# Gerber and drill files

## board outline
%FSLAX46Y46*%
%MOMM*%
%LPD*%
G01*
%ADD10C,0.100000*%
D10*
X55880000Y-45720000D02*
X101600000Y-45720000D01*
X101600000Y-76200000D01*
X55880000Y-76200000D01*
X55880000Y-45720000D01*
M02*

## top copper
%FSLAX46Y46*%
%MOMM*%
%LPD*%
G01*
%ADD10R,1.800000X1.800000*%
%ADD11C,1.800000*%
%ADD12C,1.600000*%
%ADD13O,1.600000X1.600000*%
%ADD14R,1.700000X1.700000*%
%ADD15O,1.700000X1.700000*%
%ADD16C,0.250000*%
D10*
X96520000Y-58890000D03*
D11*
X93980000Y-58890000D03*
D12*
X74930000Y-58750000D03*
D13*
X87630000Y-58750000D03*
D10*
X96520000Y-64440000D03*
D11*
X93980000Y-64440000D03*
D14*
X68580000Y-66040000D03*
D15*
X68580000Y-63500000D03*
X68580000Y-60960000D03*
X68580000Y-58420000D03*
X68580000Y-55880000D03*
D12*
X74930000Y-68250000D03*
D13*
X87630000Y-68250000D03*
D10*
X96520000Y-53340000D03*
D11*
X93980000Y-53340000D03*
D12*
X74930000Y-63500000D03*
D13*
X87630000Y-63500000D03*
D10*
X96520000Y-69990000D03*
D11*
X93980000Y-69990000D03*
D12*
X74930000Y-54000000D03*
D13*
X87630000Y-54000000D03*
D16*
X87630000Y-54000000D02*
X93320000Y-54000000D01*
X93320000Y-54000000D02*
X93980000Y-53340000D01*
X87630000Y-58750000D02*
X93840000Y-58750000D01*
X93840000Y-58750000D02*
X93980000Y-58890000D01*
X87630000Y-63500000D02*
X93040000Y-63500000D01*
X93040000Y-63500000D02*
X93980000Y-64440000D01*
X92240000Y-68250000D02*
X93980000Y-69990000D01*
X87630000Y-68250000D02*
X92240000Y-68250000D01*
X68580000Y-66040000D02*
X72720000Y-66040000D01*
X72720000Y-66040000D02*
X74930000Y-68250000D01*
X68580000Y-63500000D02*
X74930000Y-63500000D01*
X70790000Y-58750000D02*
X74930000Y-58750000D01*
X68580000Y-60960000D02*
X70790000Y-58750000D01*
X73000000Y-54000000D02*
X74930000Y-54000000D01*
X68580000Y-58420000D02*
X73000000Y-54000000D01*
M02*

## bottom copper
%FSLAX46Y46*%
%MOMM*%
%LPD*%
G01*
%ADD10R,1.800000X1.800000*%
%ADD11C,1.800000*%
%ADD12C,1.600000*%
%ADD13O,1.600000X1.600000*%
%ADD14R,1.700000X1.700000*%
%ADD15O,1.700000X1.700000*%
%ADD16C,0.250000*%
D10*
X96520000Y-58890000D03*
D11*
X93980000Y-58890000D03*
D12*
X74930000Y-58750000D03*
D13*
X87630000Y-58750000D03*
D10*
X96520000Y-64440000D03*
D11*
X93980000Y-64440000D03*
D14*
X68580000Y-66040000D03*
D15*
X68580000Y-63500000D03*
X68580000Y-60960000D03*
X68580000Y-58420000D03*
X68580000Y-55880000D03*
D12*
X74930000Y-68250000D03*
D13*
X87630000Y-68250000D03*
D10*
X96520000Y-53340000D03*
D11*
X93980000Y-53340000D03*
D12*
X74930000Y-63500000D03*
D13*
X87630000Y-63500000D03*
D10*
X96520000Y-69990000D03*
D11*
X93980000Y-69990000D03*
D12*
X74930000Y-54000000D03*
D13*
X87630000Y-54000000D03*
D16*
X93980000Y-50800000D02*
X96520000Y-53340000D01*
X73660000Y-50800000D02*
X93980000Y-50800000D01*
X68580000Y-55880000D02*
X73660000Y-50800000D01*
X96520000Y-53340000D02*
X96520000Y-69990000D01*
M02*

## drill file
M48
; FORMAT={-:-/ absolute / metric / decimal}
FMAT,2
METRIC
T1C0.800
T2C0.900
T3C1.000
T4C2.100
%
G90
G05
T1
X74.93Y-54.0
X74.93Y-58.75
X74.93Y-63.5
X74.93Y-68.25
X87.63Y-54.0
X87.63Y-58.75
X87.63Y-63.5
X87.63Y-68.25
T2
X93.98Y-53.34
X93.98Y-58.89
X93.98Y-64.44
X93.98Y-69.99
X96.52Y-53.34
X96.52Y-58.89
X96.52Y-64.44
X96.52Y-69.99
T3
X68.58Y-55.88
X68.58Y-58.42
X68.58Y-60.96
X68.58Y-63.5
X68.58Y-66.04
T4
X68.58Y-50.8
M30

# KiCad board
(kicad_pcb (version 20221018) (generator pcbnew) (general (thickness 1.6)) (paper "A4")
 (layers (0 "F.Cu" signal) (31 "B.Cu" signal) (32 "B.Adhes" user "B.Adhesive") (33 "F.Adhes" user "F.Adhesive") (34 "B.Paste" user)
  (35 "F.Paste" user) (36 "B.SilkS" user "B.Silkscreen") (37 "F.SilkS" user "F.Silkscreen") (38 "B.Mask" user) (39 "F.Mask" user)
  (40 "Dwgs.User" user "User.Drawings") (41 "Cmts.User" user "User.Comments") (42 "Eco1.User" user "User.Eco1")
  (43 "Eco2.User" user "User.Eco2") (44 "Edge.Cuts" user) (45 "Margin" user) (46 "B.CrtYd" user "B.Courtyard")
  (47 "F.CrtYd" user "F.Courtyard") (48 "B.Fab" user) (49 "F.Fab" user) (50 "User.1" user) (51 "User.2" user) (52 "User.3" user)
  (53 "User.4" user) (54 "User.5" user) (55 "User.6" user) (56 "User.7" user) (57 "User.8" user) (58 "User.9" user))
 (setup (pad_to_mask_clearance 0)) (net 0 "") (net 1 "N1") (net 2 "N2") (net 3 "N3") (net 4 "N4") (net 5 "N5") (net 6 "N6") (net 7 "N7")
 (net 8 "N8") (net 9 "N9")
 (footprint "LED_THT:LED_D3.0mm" (layer "F.Cu") (at 96.52 58.89 180)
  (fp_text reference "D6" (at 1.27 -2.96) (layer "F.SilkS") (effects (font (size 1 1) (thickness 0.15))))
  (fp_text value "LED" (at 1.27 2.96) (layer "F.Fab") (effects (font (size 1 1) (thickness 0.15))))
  (pad "1" thru_hole rect (at 0 0 180) (size 1.8 1.8) (drill 0.9) (layers "*.Cu" "*.Mask") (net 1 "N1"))
  (pad "2" thru_hole circle (at 2.54 0 180) (size 1.8 1.8) (drill 0.9) (layers "*.Cu" "*.Mask") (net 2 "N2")))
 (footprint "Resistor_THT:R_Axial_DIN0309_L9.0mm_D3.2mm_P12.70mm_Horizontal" (layer "F.Cu") (at 74.93 58.75)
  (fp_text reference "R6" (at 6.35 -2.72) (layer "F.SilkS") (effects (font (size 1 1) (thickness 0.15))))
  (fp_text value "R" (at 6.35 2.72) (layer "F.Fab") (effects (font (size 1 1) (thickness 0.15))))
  (pad "1" thru_hole circle (at 0 0) (size 1.6 1.6) (drill 0.8) (layers "*.Cu" "*.Mask") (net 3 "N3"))
  (pad "2" thru_hole oval (at 12.7 0) (size 1.6 1.6) (drill 0.8) (layers "*.Cu" "*.Mask") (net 2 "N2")))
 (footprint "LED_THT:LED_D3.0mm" (layer "F.Cu") (at 96.52 64.44 180)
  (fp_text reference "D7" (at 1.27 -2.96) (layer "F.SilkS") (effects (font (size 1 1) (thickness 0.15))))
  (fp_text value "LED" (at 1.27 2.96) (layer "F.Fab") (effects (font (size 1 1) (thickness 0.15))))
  (pad "1" thru_hole rect (at 0 0 180) (size 1.8 1.8) (drill 0.9) (layers "*.Cu" "*.Mask") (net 1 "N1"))
  (pad "2" thru_hole circle (at 2.54 0 180) (size 1.8 1.8) (drill 0.9) (layers "*.Cu" "*.Mask") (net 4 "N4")))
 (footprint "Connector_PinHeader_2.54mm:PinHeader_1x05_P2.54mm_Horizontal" (layer "F.Cu") (at 68.58 66.04 180)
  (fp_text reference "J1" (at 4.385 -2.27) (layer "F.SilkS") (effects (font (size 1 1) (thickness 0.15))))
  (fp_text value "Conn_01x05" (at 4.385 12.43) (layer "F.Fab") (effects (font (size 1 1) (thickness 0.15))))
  (pad "1" thru_hole rect (at 0 0 180) (size 1.7 1.7) (drill 1) (layers "*.Cu" "*.Mask") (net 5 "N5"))
  (pad "2" thru_hole oval (at 0 2.54 180) (size 1.7 1.7) (drill 1) (layers "*.Cu" "*.Mask") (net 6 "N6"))
  (pad "3" thru_hole oval (at 0 5.08 180) (size 1.7 1.7) (drill 1) (layers "*.Cu" "*.Mask") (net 3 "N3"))
  (pad "4" thru_hole oval (at 0 7.62 180) (size 1.7 1.7) (drill 1) (layers "*.Cu" "*.Mask") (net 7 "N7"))
  (pad "5" thru_hole oval (at 0 10.16 180) (size 1.7 1.7) (drill 1) (layers "*.Cu" "*.Mask") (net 1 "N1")))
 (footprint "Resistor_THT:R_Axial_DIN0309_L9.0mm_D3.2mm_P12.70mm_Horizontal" (layer "F.Cu") (at 74.93 68.25)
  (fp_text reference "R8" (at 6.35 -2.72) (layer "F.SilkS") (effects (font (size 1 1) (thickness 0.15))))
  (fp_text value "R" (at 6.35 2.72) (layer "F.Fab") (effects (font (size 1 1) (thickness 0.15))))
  (pad "1" thru_hole circle (at 0 0) (size 1.6 1.6) (drill 0.8) (layers "*.Cu" "*.Mask") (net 5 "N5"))
  (pad "2" thru_hole oval (at 12.7 0) (size 1.6 1.6) (drill 0.8) (layers "*.Cu" "*.Mask") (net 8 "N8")))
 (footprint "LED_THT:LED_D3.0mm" (layer "F.Cu") (at 96.52 53.34 180)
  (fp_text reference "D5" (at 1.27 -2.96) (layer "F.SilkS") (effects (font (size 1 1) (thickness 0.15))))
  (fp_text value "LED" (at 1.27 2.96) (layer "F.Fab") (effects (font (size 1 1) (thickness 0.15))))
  (pad "1" thru_hole rect (at 0 0 180) (size 1.8 1.8) (drill 0.9) (layers "*.Cu" "*.Mask") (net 1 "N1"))
  (pad "2" thru_hole circle (at 2.54 0 180) (size 1.8 1.8) (drill 0.9) (layers "*.Cu" "*.Mask") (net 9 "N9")))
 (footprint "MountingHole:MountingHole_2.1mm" (layer "F.Cu") (at 68.58 50.8)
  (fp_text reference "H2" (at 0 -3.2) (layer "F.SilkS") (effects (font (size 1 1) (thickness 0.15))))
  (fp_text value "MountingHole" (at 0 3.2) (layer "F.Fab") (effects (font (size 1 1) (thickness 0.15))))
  (pad "" np_thru_hole circle (at 0 0) (size 2.1 2.1) (drill 2.1) (layers "*.Cu" "*.Mask")))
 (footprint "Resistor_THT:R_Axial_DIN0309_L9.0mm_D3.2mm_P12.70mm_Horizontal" (layer "F.Cu") (at 74.93 63.5)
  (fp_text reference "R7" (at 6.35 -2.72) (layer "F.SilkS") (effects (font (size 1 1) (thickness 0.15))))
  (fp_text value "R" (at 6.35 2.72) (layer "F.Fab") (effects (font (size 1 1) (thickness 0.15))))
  (pad "1" thru_hole circle (at 0 0) (size 1.6 1.6) (drill 0.8) (layers "*.Cu" "*.Mask") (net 6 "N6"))
  (pad "2" thru_hole oval (at 12.7 0) (size 1.6 1.6) (drill 0.8) (layers "*.Cu" "*.Mask") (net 4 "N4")))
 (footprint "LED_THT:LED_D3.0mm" (layer "F.Cu") (at 96.52 69.99 180)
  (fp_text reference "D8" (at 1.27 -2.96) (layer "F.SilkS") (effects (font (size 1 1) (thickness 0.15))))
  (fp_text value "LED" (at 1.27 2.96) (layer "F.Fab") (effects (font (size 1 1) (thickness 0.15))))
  (pad "1" thru_hole rect (at 0 0 180) (size 1.8 1.8) (drill 0.9) (layers "*.Cu" "*.Mask") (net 1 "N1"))
  (pad "2" thru_hole circle (at 2.54 0 180) (size 1.8 1.8) (drill 0.9) (layers "*.Cu" "*.Mask") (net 8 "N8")))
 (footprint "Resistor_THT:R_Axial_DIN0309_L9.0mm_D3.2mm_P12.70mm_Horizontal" (layer "F.Cu") (at 74.93 54)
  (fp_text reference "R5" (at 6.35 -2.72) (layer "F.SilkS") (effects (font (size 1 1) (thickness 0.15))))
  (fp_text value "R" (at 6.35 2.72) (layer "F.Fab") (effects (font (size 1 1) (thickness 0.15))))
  (pad "1" thru_hole circle (at 0 0) (size 1.6 1.6) (drill 0.8) (layers "*.Cu" "*.Mask") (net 7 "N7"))
  (pad "2" thru_hole oval (at 12.7 0) (size 1.6 1.6) (drill 0.8) (layers "*.Cu" "*.Mask") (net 9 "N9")))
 (gr_rect (start 55.88 45.72) (end 101.6 76.2) (stroke (width 0.1) (type default)) (fill none) (layer "Edge.Cuts"))
 (segment (start 93.98 50.8) (end 96.52 53.34) (width 0.25) (layer "B.Cu") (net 1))
 (segment (start 73.66 50.8) (end 93.98 50.8) (width 0.25) (layer "B.Cu") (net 1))
 (segment (start 68.58 55.88) (end 73.66 50.8) (width 0.25) (layer "B.Cu") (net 1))
 (segment (start 96.52 53.34) (end 96.52 69.99) (width 0.25) (layer "B.Cu") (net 1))
 (segment (start 87.63 54) (end 93.32 54) (width 0.25) (layer "F.Cu") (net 9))
 (segment (start 93.32 54) (end 93.98 53.34) (width 0.25) (layer "F.Cu") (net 9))
 (segment (start 87.63 58.75) (end 93.84 58.75) (width 0.25) (layer "F.Cu") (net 2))
 (segment (start 93.84 58.75) (end 93.98 58.89) (width 0.25) (layer "F.Cu") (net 2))
 (segment (start 87.63 63.5) (end 93.04 63.5) (width 0.25) (layer "F.Cu") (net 4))
 (segment (start 93.04 63.5) (end 93.98 64.44) (width 0.25) (layer "F.Cu") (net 4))
 (segment (start 92.24 68.25) (end 93.98 69.99) (width 0.25) (layer "F.Cu") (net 8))
 (segment (start 87.63 68.25) (end 92.24 68.25) (width 0.25) (layer "F.Cu") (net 8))
 (segment (start 68.58 66.04) (end 72.72 66.04) (width 0.25) (layer "F.Cu") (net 5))
 (segment (start 72.72 66.04) (end 74.93 68.25) (width 0.25) (layer "F.Cu") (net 5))
 (segment (start 68.58 63.5) (end 74.93 63.5) (width 0.25) (layer "F.Cu") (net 6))
 (segment (start 70.79 58.75) (end 74.93 58.75) (width 0.25) (layer "F.Cu") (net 3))
 (segment (start 68.58 60.96) (end 70.79 58.75) (width 0.25) (layer "F.Cu") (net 3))
 (segment (start 73 54) (end 74.93 54) (width 0.25) (layer "F.Cu") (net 7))
 (segment (start 68.58 58.42) (end 73 54) (width 0.25) (layer "F.Cu") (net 7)))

